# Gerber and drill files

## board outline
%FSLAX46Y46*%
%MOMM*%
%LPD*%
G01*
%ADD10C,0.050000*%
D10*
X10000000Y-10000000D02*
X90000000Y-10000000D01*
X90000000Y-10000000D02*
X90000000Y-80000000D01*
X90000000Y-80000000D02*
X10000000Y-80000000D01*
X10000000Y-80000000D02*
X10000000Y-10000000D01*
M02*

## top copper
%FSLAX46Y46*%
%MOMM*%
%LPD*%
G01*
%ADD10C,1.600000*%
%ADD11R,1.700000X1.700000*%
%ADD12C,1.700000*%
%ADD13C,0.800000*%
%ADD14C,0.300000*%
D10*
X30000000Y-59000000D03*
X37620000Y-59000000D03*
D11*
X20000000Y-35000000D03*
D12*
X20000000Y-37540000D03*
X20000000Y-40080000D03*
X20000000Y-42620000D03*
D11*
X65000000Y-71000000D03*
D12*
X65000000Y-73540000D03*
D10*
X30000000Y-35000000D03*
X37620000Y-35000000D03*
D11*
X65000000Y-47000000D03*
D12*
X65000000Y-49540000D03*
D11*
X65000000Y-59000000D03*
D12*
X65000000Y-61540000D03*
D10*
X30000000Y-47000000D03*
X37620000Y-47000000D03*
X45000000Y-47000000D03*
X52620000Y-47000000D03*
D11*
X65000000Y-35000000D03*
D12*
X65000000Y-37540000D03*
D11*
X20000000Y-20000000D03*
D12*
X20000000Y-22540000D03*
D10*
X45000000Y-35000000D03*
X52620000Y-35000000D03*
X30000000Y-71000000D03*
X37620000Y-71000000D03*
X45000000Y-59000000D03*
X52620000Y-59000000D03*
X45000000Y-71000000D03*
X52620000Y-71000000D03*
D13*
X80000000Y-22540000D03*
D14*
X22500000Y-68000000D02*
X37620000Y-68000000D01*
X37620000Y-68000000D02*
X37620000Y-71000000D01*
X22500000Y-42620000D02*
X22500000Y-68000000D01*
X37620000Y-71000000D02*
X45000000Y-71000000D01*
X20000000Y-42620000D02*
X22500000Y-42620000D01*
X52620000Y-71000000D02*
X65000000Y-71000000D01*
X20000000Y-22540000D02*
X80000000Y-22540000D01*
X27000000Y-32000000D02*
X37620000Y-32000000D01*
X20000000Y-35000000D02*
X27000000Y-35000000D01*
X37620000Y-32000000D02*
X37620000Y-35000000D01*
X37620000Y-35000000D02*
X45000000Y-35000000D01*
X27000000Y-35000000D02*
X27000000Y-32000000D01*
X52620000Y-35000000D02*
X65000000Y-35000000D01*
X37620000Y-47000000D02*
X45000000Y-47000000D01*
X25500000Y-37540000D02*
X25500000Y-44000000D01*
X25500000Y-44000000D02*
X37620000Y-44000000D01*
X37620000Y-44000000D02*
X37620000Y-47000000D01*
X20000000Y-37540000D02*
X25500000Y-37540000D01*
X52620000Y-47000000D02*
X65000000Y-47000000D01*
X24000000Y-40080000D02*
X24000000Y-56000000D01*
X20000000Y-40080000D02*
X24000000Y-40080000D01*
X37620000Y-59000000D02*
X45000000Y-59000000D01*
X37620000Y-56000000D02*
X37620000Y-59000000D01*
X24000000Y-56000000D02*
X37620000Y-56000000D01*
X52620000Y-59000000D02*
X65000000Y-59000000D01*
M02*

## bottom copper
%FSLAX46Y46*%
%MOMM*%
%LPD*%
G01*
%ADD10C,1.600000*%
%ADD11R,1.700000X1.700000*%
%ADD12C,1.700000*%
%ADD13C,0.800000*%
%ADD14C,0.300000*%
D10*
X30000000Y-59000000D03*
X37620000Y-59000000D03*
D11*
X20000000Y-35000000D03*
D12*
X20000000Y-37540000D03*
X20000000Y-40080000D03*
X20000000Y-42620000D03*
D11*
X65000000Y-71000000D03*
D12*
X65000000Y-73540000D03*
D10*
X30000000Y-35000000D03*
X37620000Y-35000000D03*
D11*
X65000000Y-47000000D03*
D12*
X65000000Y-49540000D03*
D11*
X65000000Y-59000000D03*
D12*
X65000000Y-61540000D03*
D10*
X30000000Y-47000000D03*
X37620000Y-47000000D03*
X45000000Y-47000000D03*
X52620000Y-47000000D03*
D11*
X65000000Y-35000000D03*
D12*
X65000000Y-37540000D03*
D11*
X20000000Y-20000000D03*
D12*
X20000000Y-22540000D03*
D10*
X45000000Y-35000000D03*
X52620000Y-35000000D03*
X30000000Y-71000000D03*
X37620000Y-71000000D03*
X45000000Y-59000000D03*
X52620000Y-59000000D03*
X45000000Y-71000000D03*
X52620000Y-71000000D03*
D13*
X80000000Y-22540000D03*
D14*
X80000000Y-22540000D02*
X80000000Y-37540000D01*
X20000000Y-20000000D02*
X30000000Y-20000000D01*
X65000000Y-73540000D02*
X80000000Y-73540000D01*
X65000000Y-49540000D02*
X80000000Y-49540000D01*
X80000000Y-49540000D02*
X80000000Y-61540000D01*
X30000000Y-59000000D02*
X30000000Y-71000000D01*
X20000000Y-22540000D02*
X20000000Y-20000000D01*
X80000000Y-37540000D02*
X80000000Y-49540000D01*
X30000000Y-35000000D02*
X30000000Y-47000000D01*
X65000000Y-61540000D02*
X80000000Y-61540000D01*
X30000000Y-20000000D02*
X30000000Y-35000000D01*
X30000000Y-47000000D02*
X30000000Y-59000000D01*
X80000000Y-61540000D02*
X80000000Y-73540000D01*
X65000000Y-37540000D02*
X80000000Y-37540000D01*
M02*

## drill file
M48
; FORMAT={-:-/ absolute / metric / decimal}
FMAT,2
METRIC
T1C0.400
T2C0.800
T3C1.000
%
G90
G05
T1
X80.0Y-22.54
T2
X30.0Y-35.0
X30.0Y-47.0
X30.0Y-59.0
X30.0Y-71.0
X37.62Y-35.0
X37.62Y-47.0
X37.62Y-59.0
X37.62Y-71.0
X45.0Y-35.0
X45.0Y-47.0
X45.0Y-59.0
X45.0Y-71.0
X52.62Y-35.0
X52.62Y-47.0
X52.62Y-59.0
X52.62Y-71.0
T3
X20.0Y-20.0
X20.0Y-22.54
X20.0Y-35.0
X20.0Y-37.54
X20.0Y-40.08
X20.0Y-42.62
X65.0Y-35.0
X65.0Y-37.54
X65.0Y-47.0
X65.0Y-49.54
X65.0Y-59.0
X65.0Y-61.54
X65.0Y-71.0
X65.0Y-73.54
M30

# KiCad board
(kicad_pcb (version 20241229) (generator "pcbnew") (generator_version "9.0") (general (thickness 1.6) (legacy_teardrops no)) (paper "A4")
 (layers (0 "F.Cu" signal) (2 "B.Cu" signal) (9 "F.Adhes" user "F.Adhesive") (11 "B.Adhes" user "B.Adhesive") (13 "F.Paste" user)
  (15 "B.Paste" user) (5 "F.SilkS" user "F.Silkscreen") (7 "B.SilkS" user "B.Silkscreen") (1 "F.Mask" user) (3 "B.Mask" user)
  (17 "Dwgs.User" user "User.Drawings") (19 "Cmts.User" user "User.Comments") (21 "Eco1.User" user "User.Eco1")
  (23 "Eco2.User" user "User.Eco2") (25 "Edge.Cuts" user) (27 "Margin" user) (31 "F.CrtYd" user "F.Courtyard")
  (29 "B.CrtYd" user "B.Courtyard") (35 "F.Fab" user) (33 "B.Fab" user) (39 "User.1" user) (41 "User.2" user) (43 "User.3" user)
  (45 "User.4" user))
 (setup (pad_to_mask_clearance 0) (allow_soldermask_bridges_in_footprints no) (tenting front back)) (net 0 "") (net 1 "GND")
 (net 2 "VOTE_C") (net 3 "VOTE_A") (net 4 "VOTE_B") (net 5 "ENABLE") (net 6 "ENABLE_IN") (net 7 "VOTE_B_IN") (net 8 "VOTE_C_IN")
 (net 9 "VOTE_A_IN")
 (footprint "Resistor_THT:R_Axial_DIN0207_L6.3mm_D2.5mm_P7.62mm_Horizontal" (layer "F.Cu") (at 30 59)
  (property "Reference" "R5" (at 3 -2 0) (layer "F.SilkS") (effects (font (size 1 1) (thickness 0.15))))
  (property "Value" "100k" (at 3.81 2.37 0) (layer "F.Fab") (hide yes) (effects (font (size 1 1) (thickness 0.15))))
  (pad "1" thru_hole circle (at 0 0) (size 1.6 1.6) (drill 0.8) (layers "*.Cu" "*.Mask") (remove_unused_layers no) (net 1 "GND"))
  (pad "2" thru_hole circle (at 7.62 0) (size 1.6 1.6) (drill 0.8) (layers "*.Cu" "*.Mask") (remove_unused_layers no) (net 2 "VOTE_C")))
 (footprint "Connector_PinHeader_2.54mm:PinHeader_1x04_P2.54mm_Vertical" (layer "F.Cu") (at 20 35)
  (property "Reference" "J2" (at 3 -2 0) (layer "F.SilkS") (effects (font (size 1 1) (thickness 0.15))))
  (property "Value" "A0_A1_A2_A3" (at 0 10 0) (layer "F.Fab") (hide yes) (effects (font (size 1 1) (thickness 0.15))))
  (pad "1" thru_hole rect (at 0 0) (size 1.7 1.7) (drill 1) (layers "*.Cu" "*.Mask") (remove_unused_layers no) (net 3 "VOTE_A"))
  (pad "2" thru_hole circle (at 0 2.54) (size 1.7 1.7) (drill 1) (layers "*.Cu" "*.Mask") (remove_unused_layers no) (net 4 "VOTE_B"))
  (pad "3" thru_hole circle (at 0 5.08) (size 1.7 1.7) (drill 1) (layers "*.Cu" "*.Mask") (remove_unused_layers no) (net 2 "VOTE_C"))
  (pad "4" thru_hole circle (at 0 7.62) (size 1.7 1.7) (drill 1) (layers "*.Cu" "*.Mask") (remove_unused_layers no) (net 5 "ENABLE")))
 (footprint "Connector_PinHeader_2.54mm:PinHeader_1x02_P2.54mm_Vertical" (layer "F.Cu") (at 65 71)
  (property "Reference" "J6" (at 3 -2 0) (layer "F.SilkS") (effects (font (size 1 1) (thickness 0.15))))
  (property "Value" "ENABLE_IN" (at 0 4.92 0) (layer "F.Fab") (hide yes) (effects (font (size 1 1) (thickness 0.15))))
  (pad "1" thru_hole rect (at 0 0) (size 1.7 1.7) (drill 1) (layers "*.Cu" "*.Mask") (remove_unused_layers no) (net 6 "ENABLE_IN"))
  (pad "2" thru_hole circle (at 0 2.54) (size 1.7 1.7) (drill 1) (layers "*.Cu" "*.Mask") (remove_unused_layers no) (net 1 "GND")))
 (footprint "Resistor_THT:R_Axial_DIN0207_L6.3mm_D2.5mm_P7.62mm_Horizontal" (layer "F.Cu") (at 30 35)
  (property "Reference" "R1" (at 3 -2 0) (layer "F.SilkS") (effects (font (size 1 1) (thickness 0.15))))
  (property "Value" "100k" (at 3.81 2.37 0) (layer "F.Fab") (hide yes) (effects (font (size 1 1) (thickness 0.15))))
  (pad "1" thru_hole circle (at 0 0) (size 1.6 1.6) (drill 0.8) (layers "*.Cu" "*.Mask") (remove_unused_layers no) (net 1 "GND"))
  (pad "2" thru_hole circle (at 7.62 0) (size 1.6 1.6) (drill 0.8) (layers "*.Cu" "*.Mask") (remove_unused_layers no) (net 3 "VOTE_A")))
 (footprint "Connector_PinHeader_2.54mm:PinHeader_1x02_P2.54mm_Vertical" (layer "F.Cu") (at 65 47)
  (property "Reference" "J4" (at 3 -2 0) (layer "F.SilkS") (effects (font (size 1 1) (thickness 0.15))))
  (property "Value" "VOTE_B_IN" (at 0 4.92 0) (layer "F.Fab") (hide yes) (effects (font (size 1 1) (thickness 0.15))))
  (pad "1" thru_hole rect (at 0 0) (size 1.7 1.7) (drill 1) (layers "*.Cu" "*.Mask") (remove_unused_layers no) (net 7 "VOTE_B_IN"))
  (pad "2" thru_hole circle (at 0 2.54) (size 1.7 1.7) (drill 1) (layers "*.Cu" "*.Mask") (remove_unused_layers no) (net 1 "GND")))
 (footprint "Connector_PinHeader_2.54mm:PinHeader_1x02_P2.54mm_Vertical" (layer "F.Cu") (at 65 59)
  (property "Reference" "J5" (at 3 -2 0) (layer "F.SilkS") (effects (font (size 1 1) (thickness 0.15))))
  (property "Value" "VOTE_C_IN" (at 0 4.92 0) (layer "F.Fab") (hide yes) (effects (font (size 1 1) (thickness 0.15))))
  (pad "1" thru_hole rect (at 0 0) (size 1.7 1.7) (drill 1) (layers "*.Cu" "*.Mask") (remove_unused_layers no) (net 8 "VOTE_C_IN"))
  (pad "2" thru_hole circle (at 0 2.54) (size 1.7 1.7) (drill 1) (layers "*.Cu" "*.Mask") (remove_unused_layers no) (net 1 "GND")))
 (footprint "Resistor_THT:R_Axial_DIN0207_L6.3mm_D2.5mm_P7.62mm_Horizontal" (layer "F.Cu") (at 30 47)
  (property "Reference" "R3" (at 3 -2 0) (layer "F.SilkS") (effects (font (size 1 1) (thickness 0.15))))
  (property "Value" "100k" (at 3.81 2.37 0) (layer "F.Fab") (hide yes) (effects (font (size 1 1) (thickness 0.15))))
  (pad "1" thru_hole circle (at 0 0) (size 1.6 1.6) (drill 0.8) (layers "*.Cu" "*.Mask") (remove_unused_layers no) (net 1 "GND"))
  (pad "2" thru_hole circle (at 7.62 0) (size 1.6 1.6) (drill 0.8) (layers "*.Cu" "*.Mask") (remove_unused_layers no) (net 4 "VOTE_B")))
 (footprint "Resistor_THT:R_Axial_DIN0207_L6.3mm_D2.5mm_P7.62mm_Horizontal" (layer "F.Cu") (at 45 47)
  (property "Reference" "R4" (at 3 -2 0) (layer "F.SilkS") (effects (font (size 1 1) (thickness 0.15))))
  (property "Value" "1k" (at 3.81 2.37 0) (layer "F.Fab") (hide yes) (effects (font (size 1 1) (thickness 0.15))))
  (pad "1" thru_hole circle (at 0 0) (size 1.6 1.6) (drill 0.8) (layers "*.Cu" "*.Mask") (remove_unused_layers no) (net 4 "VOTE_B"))
  (pad "2" thru_hole circle (at 7.62 0) (size 1.6 1.6) (drill 0.8) (layers "*.Cu" "*.Mask") (remove_unused_layers no) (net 7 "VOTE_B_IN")))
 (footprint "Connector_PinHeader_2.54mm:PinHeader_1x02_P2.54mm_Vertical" (layer "F.Cu") (at 65 35)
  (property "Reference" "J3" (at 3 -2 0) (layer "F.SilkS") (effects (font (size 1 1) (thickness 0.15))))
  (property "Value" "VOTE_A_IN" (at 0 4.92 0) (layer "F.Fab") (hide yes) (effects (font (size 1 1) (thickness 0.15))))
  (pad "1" thru_hole rect (at 0 0) (size 1.7 1.7) (drill 1) (layers "*.Cu" "*.Mask") (remove_unused_layers no) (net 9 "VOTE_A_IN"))
  (pad "2" thru_hole circle (at 0 2.54) (size 1.7 1.7) (drill 1) (layers "*.Cu" "*.Mask") (remove_unused_layers no) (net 1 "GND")))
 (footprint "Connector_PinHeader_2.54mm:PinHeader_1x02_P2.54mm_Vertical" (layer "F.Cu") (at 20 20)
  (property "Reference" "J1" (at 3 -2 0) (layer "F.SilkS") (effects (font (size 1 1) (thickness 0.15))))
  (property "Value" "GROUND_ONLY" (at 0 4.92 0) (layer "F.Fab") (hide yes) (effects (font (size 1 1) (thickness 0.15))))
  (pad "1" thru_hole rect (at 0 0) (size 1.7 1.7) (drill 1) (layers "*.Cu" "*.Mask") (remove_unused_layers no) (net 1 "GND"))
  (pad "2" thru_hole circle (at 0 2.54) (size 1.7 1.7) (drill 1) (layers "*.Cu" "*.Mask") (remove_unused_layers no) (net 1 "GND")))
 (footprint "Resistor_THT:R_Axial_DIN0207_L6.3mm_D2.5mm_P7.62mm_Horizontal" (layer "F.Cu") (at 45 35)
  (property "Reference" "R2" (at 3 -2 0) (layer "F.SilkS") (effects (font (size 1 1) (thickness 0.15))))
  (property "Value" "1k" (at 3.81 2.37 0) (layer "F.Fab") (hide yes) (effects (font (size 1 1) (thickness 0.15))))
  (pad "1" thru_hole circle (at 0 0) (size 1.6 1.6) (drill 0.8) (layers "*.Cu" "*.Mask") (remove_unused_layers no) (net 3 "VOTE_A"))
  (pad "2" thru_hole circle (at 7.62 0) (size 1.6 1.6) (drill 0.8) (layers "*.Cu" "*.Mask") (remove_unused_layers no) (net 9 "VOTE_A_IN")))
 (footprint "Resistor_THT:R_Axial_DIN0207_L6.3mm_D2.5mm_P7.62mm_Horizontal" (layer "F.Cu") (at 30 71)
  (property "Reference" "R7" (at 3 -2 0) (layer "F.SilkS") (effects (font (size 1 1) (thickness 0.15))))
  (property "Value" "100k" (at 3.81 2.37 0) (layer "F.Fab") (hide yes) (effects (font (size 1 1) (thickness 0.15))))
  (pad "1" thru_hole circle (at 0 0) (size 1.6 1.6) (drill 0.8) (layers "*.Cu" "*.Mask") (remove_unused_layers no) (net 1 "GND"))
  (pad "2" thru_hole circle (at 7.62 0) (size 1.6 1.6) (drill 0.8) (layers "*.Cu" "*.Mask") (remove_unused_layers no) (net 5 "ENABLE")))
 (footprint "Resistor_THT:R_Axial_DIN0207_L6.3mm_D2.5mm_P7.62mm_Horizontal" (layer "F.Cu") (at 45 59)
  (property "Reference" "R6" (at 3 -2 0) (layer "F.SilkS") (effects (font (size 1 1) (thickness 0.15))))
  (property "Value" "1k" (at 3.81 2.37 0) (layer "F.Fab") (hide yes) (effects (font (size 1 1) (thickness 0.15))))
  (pad "1" thru_hole circle (at 0 0) (size 1.6 1.6) (drill 0.8) (layers "*.Cu" "*.Mask") (remove_unused_layers no) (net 2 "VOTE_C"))
  (pad "2" thru_hole circle (at 7.62 0) (size 1.6 1.6) (drill 0.8) (layers "*.Cu" "*.Mask") (remove_unused_layers no) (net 8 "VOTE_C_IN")))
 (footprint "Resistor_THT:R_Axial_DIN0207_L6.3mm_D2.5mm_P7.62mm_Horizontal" (layer "F.Cu") (at 45 71)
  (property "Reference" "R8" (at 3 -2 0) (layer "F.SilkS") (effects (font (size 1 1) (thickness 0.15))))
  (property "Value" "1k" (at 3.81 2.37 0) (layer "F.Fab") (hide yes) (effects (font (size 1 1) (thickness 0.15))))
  (pad "1" thru_hole circle (at 0 0) (size 1.6 1.6) (drill 0.8) (layers "*.Cu" "*.Mask") (remove_unused_layers no) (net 5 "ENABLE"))
  (pad "2" thru_hole circle (at 7.62 0) (size 1.6 1.6) (drill 0.8) (layers "*.Cu" "*.Mask") (remove_unused_layers no) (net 6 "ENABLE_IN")))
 (gr_line (start 10 10) (end 90 10) (stroke (width 0.05) (type default)) (layer "Edge.Cuts"))
 (gr_line (start 90 10) (end 90 80) (stroke (width 0.05) (type default)) (layer "Edge.Cuts"))
 (gr_line (start 90 80) (end 10 80) (stroke (width 0.05) (type default)) (layer "Edge.Cuts"))
 (gr_line (start 10 80) (end 10 10) (stroke (width 0.05) (type default)) (layer "Edge.Cuts"))
 (segment (start 22.5 68) (end 37.62 68) (width 0.3) (layer "F.Cu") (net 5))
 (segment (start 37.62 68) (end 37.62 71) (width 0.3) (layer "F.Cu") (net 5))
 (segment (start 22.5 42.62) (end 22.5 68) (width 0.3) (layer "F.Cu") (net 5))
 (segment (start 37.62 71) (end 45 71) (width 0.3) (layer "F.Cu") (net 5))
 (segment (start 20 42.62) (end 22.5 42.62) (width 0.3) (layer "F.Cu") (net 5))
 (segment (start 52.62 71) (end 65 71) (width 0.3) (layer "F.Cu") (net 6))
 (segment (start 20 22.54) (end 80 22.54) (width 0.3) (layer "F.Cu") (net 1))
 (via (at 80 22.54) (size 0.8) (drill 0.4) (layers "F.Cu" "B.Cu") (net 1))
 (segment (start 80 22.54) (end 80 37.54) (width 0.3) (layer "B.Cu") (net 1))
 (segment (start 20 20) (end 30 20) (width 0.3) (layer "B.Cu") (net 1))
 (segment (start 65 73.54) (end 80 73.54) (width 0.3) (layer "B.Cu") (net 1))
 (segment (start 65 49.54) (end 80 49.54) (width 0.3) (layer "B.Cu") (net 1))
 (segment (start 80 49.54) (end 80 61.54) (width 0.3) (layer "B.Cu") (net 1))
 (segment (start 30 59) (end 30 71) (width 0.3) (layer "B.Cu") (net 1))
 (segment (start 20 22.54) (end 20 20) (width 0.3) (layer "B.Cu") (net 1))
 (segment (start 80 37.54) (end 80 49.54) (width 0.3) (layer "B.Cu") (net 1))
 (segment (start 30 35) (end 30 47) (width 0.3) (layer "B.Cu") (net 1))
 (segment (start 65 61.54) (end 80 61.54) (width 0.3) (layer "B.Cu") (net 1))
 (segment (start 30 20) (end 30 35) (width 0.3) (layer "B.Cu") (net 1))
 (segment (start 30 47) (end 30 59) (width 0.3) (layer "B.Cu") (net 1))
 (segment (start 80 61.54) (end 80 73.54) (width 0.3) (layer "B.Cu") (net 1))
 (segment (start 65 37.54) (end 80 37.54) (width 0.3) (layer "B.Cu") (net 1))
 (segment (start 27 32) (end 37.62 32) (width 0.3) (layer "F.Cu") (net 3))
 (segment (start 20 35) (end 27 35) (width 0.3) (layer "F.Cu") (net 3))
 (segment (start 37.62 32) (end 37.62 35) (width 0.3) (layer "F.Cu") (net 3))
 (segment (start 37.62 35) (end 45 35) (width 0.3) (layer "F.Cu") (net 3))
 (segment (start 27 35) (end 27 32) (width 0.3) (layer "F.Cu") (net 3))
 (segment (start 52.62 35) (end 65 35) (width 0.3) (layer "F.Cu") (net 9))
 (segment (start 37.62 47) (end 45 47) (width 0.3) (layer "F.Cu") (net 4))
 (segment (start 25.5 37.54) (end 25.5 44) (width 0.3) (layer "F.Cu") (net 4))
 (segment (start 25.5 44) (end 37.62 44) (width 0.3) (layer "F.Cu") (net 4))
 (segment (start 37.62 44) (end 37.62 47) (width 0.3) (layer "F.Cu") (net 4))
 (segment (start 20 37.54) (end 25.5 37.54) (width 0.3) (layer "F.Cu") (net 4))
 (segment (start 52.62 47) (end 65 47) (width 0.3) (layer "F.Cu") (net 7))
 (segment (start 24 40.08) (end 24 56) (width 0.3) (layer "F.Cu") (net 2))
 (segment (start 20 40.08) (end 24 40.08) (width 0.3) (layer "F.Cu") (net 2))
 (segment (start 37.62 59) (end 45 59) (width 0.3) (layer "F.Cu") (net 2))
 (segment (start 37.62 56) (end 37.62 59) (width 0.3) (layer "F.Cu") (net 2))
 (segment (start 24 56) (end 37.62 56) (width 0.3) (layer "F.Cu") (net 2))
 (segment (start 52.62 59) (end 65 59) (width 0.3) (layer "F.Cu") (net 8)))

